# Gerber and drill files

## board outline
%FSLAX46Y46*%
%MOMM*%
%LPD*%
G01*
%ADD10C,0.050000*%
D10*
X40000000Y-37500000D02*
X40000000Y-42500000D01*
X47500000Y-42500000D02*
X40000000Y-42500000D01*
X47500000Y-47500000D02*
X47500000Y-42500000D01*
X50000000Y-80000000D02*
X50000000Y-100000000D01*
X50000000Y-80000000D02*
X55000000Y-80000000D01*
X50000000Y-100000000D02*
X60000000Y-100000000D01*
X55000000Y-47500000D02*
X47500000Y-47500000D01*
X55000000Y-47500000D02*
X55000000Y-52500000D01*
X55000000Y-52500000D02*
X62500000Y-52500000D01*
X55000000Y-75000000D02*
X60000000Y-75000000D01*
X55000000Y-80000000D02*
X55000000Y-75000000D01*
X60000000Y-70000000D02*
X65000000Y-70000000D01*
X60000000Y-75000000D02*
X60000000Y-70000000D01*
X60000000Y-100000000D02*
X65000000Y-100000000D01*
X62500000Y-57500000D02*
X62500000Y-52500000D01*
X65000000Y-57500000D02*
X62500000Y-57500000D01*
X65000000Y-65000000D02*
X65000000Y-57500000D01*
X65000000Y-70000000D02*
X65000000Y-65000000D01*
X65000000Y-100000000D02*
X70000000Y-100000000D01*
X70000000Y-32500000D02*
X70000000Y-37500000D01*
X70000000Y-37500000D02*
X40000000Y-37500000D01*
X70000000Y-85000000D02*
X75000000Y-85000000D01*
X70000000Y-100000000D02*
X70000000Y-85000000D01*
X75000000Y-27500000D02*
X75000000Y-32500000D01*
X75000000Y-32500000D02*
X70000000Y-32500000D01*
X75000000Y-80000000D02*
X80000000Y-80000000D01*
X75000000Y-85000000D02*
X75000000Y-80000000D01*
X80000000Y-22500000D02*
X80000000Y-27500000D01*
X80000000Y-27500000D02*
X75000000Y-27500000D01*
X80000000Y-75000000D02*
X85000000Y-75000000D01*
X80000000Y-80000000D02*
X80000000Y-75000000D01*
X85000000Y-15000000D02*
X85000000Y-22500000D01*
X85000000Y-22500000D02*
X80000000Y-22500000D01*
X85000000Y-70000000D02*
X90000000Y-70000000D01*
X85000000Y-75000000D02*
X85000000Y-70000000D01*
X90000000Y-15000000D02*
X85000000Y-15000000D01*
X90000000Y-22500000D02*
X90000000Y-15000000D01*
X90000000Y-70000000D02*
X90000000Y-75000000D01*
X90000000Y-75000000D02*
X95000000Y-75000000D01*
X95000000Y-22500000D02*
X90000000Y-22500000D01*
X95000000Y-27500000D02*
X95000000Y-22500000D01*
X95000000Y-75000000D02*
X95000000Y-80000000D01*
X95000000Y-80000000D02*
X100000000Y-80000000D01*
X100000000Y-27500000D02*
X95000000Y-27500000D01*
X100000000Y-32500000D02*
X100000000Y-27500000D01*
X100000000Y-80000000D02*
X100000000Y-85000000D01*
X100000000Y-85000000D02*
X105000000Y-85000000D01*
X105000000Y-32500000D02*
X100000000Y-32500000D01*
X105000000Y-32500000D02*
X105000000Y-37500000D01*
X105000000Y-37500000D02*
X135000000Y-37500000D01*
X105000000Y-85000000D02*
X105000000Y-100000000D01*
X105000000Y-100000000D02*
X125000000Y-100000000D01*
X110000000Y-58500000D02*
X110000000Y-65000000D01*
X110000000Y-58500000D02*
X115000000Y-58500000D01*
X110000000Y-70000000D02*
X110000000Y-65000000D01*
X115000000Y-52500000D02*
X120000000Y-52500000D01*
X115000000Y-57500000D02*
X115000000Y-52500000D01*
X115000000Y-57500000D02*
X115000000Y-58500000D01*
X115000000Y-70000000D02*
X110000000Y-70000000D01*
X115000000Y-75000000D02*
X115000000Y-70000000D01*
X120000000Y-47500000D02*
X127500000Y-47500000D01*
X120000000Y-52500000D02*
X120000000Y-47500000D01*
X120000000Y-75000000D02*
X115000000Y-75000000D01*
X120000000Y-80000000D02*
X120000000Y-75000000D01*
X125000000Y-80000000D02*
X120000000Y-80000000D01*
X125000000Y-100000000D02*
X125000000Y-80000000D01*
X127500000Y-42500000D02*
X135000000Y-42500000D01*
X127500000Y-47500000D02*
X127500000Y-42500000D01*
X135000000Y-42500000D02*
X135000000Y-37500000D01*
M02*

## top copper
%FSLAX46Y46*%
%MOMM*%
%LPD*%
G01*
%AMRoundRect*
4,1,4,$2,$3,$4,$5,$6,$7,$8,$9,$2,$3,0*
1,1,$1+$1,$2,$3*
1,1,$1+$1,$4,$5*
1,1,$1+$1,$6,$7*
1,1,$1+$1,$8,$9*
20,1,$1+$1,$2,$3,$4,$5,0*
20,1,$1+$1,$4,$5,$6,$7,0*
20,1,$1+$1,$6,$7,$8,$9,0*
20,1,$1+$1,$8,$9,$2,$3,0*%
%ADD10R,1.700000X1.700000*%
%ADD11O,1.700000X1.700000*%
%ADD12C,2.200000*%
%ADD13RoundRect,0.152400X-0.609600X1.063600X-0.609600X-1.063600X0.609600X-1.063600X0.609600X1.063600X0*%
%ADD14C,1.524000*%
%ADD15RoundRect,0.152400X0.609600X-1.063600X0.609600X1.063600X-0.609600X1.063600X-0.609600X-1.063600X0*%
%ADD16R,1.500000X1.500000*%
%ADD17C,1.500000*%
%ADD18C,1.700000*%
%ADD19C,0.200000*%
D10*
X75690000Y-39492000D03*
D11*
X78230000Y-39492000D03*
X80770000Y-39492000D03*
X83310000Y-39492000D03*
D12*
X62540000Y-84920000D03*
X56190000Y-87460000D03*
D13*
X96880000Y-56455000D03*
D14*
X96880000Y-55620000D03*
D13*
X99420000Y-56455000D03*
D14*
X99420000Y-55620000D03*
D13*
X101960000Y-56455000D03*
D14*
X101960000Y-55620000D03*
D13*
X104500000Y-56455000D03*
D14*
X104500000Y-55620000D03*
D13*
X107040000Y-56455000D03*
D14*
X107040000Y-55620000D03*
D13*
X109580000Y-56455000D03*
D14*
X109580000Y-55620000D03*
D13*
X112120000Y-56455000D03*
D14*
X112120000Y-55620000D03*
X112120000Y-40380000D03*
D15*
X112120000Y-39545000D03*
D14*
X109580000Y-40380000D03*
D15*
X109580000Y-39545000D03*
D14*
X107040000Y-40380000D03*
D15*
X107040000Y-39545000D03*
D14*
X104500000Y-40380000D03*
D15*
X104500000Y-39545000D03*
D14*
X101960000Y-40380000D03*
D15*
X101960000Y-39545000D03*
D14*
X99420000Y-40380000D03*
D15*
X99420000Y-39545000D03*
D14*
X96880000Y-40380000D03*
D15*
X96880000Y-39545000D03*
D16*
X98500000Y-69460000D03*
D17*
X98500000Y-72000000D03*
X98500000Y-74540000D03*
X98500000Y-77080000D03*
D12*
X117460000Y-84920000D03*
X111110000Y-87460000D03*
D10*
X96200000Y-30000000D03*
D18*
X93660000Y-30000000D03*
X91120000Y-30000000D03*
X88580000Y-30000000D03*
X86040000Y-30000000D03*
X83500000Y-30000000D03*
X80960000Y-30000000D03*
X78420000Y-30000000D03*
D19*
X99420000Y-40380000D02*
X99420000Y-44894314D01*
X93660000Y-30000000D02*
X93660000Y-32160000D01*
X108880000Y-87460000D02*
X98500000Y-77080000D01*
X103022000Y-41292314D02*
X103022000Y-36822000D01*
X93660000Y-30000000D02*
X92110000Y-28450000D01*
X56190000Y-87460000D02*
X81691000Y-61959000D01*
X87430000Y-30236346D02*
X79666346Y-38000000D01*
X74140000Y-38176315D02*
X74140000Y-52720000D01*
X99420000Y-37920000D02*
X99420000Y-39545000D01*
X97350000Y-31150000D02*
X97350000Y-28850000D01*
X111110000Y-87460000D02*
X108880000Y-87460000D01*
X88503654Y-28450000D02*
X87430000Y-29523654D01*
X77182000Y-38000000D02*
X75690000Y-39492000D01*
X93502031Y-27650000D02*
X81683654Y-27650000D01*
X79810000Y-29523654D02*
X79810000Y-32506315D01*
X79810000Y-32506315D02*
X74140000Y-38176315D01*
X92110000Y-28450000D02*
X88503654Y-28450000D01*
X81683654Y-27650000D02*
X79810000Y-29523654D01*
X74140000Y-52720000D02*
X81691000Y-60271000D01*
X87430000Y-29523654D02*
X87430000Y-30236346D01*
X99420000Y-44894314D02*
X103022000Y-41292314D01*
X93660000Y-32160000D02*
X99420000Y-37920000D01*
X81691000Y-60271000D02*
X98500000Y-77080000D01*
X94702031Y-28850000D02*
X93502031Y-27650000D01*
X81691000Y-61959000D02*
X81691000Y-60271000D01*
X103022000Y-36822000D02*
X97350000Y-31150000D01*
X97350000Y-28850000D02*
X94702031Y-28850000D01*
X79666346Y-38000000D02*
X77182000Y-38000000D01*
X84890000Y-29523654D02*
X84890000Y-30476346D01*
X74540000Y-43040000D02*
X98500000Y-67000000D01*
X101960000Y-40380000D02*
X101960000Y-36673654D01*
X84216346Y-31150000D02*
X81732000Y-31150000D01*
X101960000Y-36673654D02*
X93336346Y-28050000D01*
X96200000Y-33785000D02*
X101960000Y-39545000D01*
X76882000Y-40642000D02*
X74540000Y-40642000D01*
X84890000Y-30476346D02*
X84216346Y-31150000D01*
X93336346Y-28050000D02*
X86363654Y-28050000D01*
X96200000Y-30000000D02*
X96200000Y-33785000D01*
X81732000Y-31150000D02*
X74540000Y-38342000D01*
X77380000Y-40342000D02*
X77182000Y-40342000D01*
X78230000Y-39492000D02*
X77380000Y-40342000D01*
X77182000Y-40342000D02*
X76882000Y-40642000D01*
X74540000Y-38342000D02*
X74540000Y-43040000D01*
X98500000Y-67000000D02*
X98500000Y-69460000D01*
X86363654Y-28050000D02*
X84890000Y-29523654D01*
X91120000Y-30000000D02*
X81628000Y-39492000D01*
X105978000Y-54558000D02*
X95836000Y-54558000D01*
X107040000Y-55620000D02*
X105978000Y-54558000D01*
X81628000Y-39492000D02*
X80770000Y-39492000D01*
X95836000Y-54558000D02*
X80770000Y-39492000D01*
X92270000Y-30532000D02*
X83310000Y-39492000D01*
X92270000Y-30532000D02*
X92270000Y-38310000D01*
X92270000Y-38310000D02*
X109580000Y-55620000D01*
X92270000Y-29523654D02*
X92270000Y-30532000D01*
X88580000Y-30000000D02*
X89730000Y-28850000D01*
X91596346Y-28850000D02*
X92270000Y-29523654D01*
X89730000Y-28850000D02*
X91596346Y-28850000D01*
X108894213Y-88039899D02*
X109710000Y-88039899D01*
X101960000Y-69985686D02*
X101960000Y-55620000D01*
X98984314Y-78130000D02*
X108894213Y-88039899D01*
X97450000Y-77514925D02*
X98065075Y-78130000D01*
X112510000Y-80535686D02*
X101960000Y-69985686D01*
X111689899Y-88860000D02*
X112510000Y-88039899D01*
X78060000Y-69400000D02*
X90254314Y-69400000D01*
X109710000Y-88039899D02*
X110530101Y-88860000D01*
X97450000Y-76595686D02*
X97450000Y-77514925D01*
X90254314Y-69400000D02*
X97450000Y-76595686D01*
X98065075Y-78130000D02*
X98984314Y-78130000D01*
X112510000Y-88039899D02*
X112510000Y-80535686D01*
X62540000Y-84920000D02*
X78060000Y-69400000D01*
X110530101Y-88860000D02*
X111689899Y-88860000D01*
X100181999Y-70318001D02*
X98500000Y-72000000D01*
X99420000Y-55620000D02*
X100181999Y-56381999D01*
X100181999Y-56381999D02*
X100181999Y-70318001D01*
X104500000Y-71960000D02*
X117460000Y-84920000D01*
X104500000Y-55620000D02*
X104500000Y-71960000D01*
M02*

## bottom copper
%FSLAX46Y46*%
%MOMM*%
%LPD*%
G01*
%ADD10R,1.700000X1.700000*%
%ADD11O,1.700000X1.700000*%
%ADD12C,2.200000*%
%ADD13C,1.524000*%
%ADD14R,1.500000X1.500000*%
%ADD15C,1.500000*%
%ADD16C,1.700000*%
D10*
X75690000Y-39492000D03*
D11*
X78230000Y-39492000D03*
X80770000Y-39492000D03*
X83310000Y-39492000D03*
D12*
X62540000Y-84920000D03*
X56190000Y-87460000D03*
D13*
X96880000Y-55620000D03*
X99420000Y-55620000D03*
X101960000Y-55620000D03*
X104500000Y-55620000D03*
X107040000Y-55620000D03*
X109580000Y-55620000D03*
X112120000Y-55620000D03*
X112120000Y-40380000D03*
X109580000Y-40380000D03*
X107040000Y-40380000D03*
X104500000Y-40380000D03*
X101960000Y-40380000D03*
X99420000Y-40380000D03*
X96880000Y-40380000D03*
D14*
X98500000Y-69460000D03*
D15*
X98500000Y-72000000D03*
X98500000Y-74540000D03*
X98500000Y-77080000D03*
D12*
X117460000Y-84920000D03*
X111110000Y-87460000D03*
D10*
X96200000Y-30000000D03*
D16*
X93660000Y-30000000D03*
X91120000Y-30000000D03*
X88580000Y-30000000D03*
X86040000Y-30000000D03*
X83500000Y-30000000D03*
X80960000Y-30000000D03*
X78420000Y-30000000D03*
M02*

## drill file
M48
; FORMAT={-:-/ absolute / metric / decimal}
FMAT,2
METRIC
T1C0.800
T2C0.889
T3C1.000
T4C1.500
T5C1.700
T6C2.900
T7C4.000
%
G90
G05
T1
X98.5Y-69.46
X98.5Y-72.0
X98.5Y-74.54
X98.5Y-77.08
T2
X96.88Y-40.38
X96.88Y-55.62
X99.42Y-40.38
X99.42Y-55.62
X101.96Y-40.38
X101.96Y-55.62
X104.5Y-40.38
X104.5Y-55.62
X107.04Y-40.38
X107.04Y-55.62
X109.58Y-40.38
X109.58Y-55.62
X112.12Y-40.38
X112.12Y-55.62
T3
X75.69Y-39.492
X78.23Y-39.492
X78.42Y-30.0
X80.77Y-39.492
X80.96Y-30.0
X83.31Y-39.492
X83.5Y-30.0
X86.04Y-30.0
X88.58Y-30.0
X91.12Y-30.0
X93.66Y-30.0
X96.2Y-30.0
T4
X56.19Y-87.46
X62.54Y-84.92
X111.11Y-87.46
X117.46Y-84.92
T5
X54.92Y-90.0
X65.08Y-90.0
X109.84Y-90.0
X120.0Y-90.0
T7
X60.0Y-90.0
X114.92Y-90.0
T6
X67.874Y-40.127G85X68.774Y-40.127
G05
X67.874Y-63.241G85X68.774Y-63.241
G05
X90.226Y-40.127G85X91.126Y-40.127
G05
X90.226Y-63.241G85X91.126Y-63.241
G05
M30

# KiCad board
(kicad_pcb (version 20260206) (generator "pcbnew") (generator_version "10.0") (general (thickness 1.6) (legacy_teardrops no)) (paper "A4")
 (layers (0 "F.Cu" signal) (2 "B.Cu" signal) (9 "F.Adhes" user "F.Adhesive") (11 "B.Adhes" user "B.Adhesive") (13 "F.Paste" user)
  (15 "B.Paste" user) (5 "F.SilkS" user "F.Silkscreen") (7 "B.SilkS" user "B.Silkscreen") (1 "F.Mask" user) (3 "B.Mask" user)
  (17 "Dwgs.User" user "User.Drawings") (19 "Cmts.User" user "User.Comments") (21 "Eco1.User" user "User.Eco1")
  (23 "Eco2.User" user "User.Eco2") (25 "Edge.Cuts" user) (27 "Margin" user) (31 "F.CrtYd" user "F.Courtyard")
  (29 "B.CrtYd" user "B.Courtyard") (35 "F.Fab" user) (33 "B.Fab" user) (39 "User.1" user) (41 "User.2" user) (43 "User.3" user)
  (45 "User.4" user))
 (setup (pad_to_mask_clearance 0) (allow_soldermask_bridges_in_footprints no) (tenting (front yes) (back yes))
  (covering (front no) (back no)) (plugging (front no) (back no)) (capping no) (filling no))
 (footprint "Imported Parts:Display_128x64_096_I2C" (layer "F.Cu") (at 79.5 39.492)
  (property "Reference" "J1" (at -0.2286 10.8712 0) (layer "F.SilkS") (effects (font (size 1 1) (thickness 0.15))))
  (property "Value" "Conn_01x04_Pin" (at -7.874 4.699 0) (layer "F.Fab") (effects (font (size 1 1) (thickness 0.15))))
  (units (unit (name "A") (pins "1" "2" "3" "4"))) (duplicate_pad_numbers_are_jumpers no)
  (pad "" np_thru_hole oval (at -11.176 0.635) (size 3.8 2.9) (drill oval 3.8 2.9) (layers "*.Cu" "*.Mask"))
  (pad "" np_thru_hole oval (at -11.176 23.749) (size 3.8 2.9) (drill oval 3.8 2.9) (layers "*.Cu" "*.Mask"))
  (pad "" np_thru_hole oval (at 11.176 0.635) (size 3.8 2.9) (drill oval 3.8 2.9) (layers "*.Cu" "*.Mask"))
  (pad "" np_thru_hole oval (at 11.176 23.749) (size 3.8 2.9) (drill oval 3.8 2.9) (layers "*.Cu" "*.Mask"))
  (pad "1" thru_hole rect (at -3.81 0 90) (size 1.7 1.7) (drill 1) (layers "*.Cu" "*.Mask") (remove_unused_layers no) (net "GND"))
  (pad "2" thru_hole oval (at -1.27 0 90) (size 1.7 1.7) (drill 1) (layers "*.Cu" "*.Mask") (remove_unused_layers no) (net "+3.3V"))
  (pad "3" thru_hole oval (at 1.27 0 90) (size 1.7 1.7) (drill 1) (layers "*.Cu" "*.Mask") (remove_unused_layers no) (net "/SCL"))
  (pad "4" thru_hole oval (at 3.81 0 90) (size 1.7 1.7) (drill 1) (layers "*.Cu" "*.Mask") (remove_unused_layers no) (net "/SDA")))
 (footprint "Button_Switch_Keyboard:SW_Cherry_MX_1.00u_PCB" (layer "F.Cu") (at 62.54 84.92)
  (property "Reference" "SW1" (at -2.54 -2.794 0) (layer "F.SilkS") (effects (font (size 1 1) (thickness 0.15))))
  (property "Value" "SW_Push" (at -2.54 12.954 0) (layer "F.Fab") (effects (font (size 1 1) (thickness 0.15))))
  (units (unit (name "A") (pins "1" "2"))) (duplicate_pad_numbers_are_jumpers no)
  (pad "" np_thru_hole circle (at -7.62 5.08) (size 1.7 1.7) (drill 1.7) (layers "*.Cu" "*.Mask"))
  (pad "" np_thru_hole circle (at -2.54 5.08) (size 4 4) (drill 4) (layers "*.Cu" "*.Mask"))
  (pad "" np_thru_hole circle (at 2.54 5.08) (size 1.7 1.7) (drill 1.7) (layers "*.Cu" "*.Mask"))
  (pad "1" thru_hole circle (at 0 0) (size 2.2 2.2) (drill 1.5) (layers "*.Cu" "*.Mask") (remove_unused_layers no) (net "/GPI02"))
  (pad "2" thru_hole circle (at -6.35 2.54) (size 2.2 2.2) (drill 1.5) (layers "*.Cu" "*.Mask") (remove_unused_layers no) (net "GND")))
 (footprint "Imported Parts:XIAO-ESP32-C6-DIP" (layer "F.Cu") (at 104.5 48 180)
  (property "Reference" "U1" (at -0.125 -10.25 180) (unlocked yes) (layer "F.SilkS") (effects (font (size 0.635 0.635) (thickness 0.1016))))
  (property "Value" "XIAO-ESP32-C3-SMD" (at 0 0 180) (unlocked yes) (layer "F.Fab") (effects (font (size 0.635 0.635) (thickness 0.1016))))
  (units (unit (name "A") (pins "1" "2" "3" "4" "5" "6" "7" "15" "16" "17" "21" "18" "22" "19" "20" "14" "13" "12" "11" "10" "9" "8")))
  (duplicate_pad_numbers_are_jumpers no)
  (pad "1" smd roundrect (at 7.62 -8.455 270) (size 2.432 1.524) (layers "F.Cu" "F.Mask") (roundrect_rratio 0.1)
   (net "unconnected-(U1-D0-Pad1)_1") (thermal_bridge_angle 45))
  (pad "1" thru_hole circle (at 7.62 -7.62 270) (size 1.524 1.524) (drill 0.889) (layers "*.Cu" "*.Mask") (remove_unused_layers no)
   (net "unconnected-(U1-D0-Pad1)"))
  (pad "2" smd roundrect (at 5.08 -8.455 270) (size 2.432 1.524) (layers "F.Cu" "F.Mask") (roundrect_rratio 0.1) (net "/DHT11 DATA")
   (thermal_bridge_angle 45))
  (pad "2" thru_hole circle (at 5.08 -7.62 270) (size 1.524 1.524) (drill 0.889) (layers "*.Cu" "*.Mask") (remove_unused_layers no)
   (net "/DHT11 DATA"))
  (pad "3" smd roundrect (at 2.54 -8.455 270) (size 2.432 1.524) (layers "F.Cu" "F.Mask") (roundrect_rratio 0.1) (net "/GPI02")
   (thermal_bridge_angle 45))
  (pad "3" thru_hole circle (at 2.54 -7.62 270) (size 1.524 1.524) (drill 0.889) (layers "*.Cu" "*.Mask") (remove_unused_layers no)
   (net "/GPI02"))
  (pad "4" smd roundrect (at 0 -8.455 270) (size 2.432 1.524) (layers "F.Cu" "F.Mask") (roundrect_rratio 0.1) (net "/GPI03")
   (thermal_bridge_angle 45))
  (pad "4" thru_hole circle (at 0 -7.62 270) (size 1.524 1.524) (drill 0.889) (layers "*.Cu" "*.Mask") (remove_unused_layers no)
   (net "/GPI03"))
  (pad "5" smd roundrect (at -2.54 -8.455 270) (size 2.432 1.524) (layers "F.Cu" "F.Mask") (roundrect_rratio 0.1) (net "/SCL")
   (thermal_bridge_angle 45))
  (pad "5" thru_hole circle (at -2.54 -7.62 270) (size 1.524 1.524) (drill 0.889) (layers "*.Cu" "*.Mask") (remove_unused_layers no)
   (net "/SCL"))
  (pad "6" smd roundrect (at -5.08 -8.455 270) (size 2.432 1.524) (layers "F.Cu" "F.Mask") (roundrect_rratio 0.1) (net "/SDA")
   (thermal_bridge_angle 45))
  (pad "6" thru_hole circle (at -5.08 -7.62 270) (size 1.524 1.524) (drill 0.889) (layers "*.Cu" "*.Mask") (remove_unused_layers no)
   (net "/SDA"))
  (pad "7" smd roundrect (at -7.62 -8.455 270) (size 2.432 1.524) (layers "F.Cu" "F.Mask") (roundrect_rratio 0.1)
   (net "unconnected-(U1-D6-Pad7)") (thermal_bridge_angle 45))
  (pad "7" thru_hole circle (at -7.62 -7.62 270) (size 1.524 1.524) (drill 0.889) (layers "*.Cu" "*.Mask") (remove_unused_layers no)
   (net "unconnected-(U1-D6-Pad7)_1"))
  (pad "8" thru_hole circle (at -7.62 7.62 90) (size 1.524 1.524) (drill 0.889) (layers "*.Cu" "*.Mask") (remove_unused_layers no)
   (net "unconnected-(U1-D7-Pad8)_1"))
  (pad "8" smd roundrect (at -7.62 8.455 90) (size 2.432 1.524) (layers "F.Cu" "F.Mask") (roundrect_rratio 0.1)
   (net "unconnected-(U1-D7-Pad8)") (thermal_bridge_angle 45))
  (pad "9" thru_hole circle (at -5.08 7.62 90) (size 1.524 1.524) (drill 0.889) (layers "*.Cu" "*.Mask") (remove_unused_layers no)
   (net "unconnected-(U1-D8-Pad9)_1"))
  (pad "9" smd roundrect (at -5.08 8.455 90) (size 2.432 1.524) (layers "F.Cu" "F.Mask") (roundrect_rratio 0.1)
   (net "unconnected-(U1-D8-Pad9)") (thermal_bridge_angle 45))
  (pad "10" thru_hole circle (at -2.54 7.62 90) (size 1.524 1.524) (drill 0.889) (layers "*.Cu" "*.Mask") (remove_unused_layers no)
   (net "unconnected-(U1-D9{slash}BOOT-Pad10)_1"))
  (pad "10" smd roundrect (at -2.54 8.455 90) (size 2.432 1.524) (layers "F.Cu" "F.Mask") (roundrect_rratio 0.1)
   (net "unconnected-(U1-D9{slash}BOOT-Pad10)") (thermal_bridge_angle 45))
  (pad "11" thru_hole circle (at 0 7.62 90) (size 1.524 1.524) (drill 0.889) (layers "*.Cu" "*.Mask") (remove_unused_layers no)
   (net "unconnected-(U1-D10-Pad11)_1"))
  (pad "11" smd roundrect (at 0 8.455 90) (size 2.432 1.524) (layers "F.Cu" "F.Mask") (roundrect_rratio 0.1)
   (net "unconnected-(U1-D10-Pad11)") (thermal_bridge_angle 45))
  (pad "12" thru_hole circle (at 2.54 7.62 90) (size 1.524 1.524) (drill 0.889) (layers "*.Cu" "*.Mask") (remove_unused_layers no)
   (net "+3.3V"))
  (pad "12" smd roundrect (at 2.54 8.455 90) (size 2.432 1.524) (layers "F.Cu" "F.Mask") (roundrect_rratio 0.1) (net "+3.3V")
   (thermal_bridge_angle 45))
  (pad "13" thru_hole circle (at 5.08 7.62 90) (size 1.524 1.524) (drill 0.889) (layers "*.Cu" "*.Mask") (remove_unused_layers no)
   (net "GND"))
  (pad "13" smd roundrect (at 5.08 8.455 90) (size 2.432 1.524) (layers "F.Cu" "F.Mask") (roundrect_rratio 0.1) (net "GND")
   (thermal_bridge_angle 45))
  (pad "14" thru_hole circle (at 7.62 7.62 90) (size 1.524 1.524) (drill 0.889) (layers "*.Cu" "*.Mask") (remove_unused_layers no)
   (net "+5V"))
  (pad "14" smd roundrect (at 7.62 8.455 90) (size 2.432 1.524) (layers "F.Cu" "F.Mask") (roundrect_rratio 0.1) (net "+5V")
   (thermal_bridge_angle 45)))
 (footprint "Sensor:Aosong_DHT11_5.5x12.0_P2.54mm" (layer "F.Cu") (at 98.5 69.46)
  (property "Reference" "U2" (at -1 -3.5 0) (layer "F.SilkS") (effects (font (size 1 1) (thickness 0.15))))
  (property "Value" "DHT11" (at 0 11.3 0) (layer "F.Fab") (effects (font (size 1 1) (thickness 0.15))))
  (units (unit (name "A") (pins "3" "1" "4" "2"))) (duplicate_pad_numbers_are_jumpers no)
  (pad "1" thru_hole rect (at 0 0) (size 1.5 1.5) (drill 0.8) (layers "*.Cu" "*.Mask") (remove_unused_layers no) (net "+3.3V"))
  (pad "2" thru_hole circle (at 0 2.54) (size 1.5 1.5) (drill 0.8) (layers "*.Cu" "*.Mask") (remove_unused_layers no) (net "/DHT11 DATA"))
  (pad "3" thru_hole circle (at 0 5.08) (size 1.5 1.5) (drill 0.8) (layers "*.Cu" "*.Mask") (remove_unused_layers no)
   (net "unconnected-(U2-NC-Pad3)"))
  (pad "4" thru_hole circle (at 0 7.62) (size 1.5 1.5) (drill 0.8) (layers "*.Cu" "*.Mask") (remove_unused_layers no) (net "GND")))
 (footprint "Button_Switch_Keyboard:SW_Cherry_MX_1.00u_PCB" (layer "F.Cu") (at 117.46 84.92)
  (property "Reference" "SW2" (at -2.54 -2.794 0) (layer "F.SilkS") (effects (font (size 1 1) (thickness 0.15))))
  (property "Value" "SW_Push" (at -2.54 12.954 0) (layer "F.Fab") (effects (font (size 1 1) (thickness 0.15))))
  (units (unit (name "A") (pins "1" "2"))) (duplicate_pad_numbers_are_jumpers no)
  (pad "" np_thru_hole circle (at -7.62 5.08) (size 1.7 1.7) (drill 1.7) (layers "*.Cu" "*.Mask"))
  (pad "" np_thru_hole circle (at -2.54 5.08) (size 4 4) (drill 4) (layers "*.Cu" "*.Mask"))
  (pad "" np_thru_hole circle (at 2.54 5.08) (size 1.7 1.7) (drill 1.7) (layers "*.Cu" "*.Mask"))
  (pad "1" thru_hole circle (at 0 0) (size 2.2 2.2) (drill 1.5) (layers "*.Cu" "*.Mask") (remove_unused_layers no) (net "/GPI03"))
  (pad "2" thru_hole circle (at -6.35 2.54) (size 2.2 2.2) (drill 1.5) (layers "*.Cu" "*.Mask") (remove_unused_layers no) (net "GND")))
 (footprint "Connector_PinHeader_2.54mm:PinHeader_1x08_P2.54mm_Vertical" (layer "F.Cu") (at 96.2 30 -90)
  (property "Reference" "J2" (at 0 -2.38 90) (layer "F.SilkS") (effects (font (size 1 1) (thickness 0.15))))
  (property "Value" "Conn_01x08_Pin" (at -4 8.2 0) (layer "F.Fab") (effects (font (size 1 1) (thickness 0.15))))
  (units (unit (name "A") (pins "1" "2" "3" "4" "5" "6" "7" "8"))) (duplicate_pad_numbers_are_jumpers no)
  (pad "1" thru_hole rect (at 0 0 270) (size 1.7 1.7) (drill 1) (layers "*.Cu" "*.Mask") (remove_unused_layers no) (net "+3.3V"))
  (pad "2" thru_hole circle (at 0 2.54 270) (size 1.7 1.7) (drill 1) (layers "*.Cu" "*.Mask") (remove_unused_layers no) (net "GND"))
  (pad "3" thru_hole circle (at 0 5.08 270) (size 1.7 1.7) (drill 1) (layers "*.Cu" "*.Mask") (remove_unused_layers no) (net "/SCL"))
  (pad "4" thru_hole circle (at 0 7.62 270) (size 1.7 1.7) (drill 1) (layers "*.Cu" "*.Mask") (remove_unused_layers no) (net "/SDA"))
  (pad "5" thru_hole circle (at 0 10.16 270) (size 1.7 1.7) (drill 1) (layers "*.Cu" "*.Mask") (remove_unused_layers no)
   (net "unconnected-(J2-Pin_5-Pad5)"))
  (pad "6" thru_hole circle (at 0 12.7 270) (size 1.7 1.7) (drill 1) (layers "*.Cu" "*.Mask") (remove_unused_layers no)
   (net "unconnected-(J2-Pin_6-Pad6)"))
  (pad "7" thru_hole circle (at 0 15.24 270) (size 1.7 1.7) (drill 1) (layers "*.Cu" "*.Mask") (remove_unused_layers no)
   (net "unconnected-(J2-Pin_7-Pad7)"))
  (pad "8" thru_hole circle (at 0 17.78 270) (size 1.7 1.7) (drill 1) (layers "*.Cu" "*.Mask") (remove_unused_layers no)
   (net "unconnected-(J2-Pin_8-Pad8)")))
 (gr_line (start 40 37.5) (end 40 42.5) (stroke (width 0.05) (type default)) (layer "Edge.Cuts"))
 (gr_line (start 47.5 42.5) (end 40 42.5) (stroke (width 0.05) (type default)) (layer "Edge.Cuts"))
 (gr_line (start 47.5 47.5) (end 47.5 42.5) (stroke (width 0.05) (type default)) (layer "Edge.Cuts"))
 (gr_line (start 50 80) (end 50 100) (stroke (width 0.05) (type default)) (layer "Edge.Cuts"))
 (gr_line (start 50 80) (end 55 80) (stroke (width 0.05) (type default)) (layer "Edge.Cuts"))
 (gr_line (start 50 100) (end 60 100) (stroke (width 0.05) (type default)) (layer "Edge.Cuts"))
 (gr_line (start 55 47.5) (end 47.5 47.5) (stroke (width 0.05) (type default)) (layer "Edge.Cuts"))
 (gr_line (start 55 47.5) (end 55 52.5) (stroke (width 0.05) (type default)) (layer "Edge.Cuts"))
 (gr_line (start 55 52.5) (end 62.5 52.5) (stroke (width 0.05) (type default)) (layer "Edge.Cuts"))
 (gr_line (start 55 75) (end 60 75) (stroke (width 0.05) (type default)) (layer "Edge.Cuts"))
 (gr_line (start 55 80) (end 55 75) (stroke (width 0.05) (type default)) (layer "Edge.Cuts"))
 (gr_line (start 60 70) (end 65 70) (stroke (width 0.05) (type default)) (layer "Edge.Cuts"))
 (gr_line (start 60 75) (end 60 70) (stroke (width 0.05) (type default)) (layer "Edge.Cuts"))
 (gr_line (start 60 100) (end 65 100) (stroke (width 0.05) (type default)) (layer "Edge.Cuts"))
 (gr_line (start 62.5 57.5) (end 62.5 52.5) (stroke (width 0.05) (type default)) (layer "Edge.Cuts"))
 (gr_line (start 65 57.5) (end 62.5 57.5) (stroke (width 0.05) (type default)) (layer "Edge.Cuts"))
 (gr_line (start 65 65) (end 65 57.5) (stroke (width 0.05) (type default)) (layer "Edge.Cuts"))
 (gr_line (start 65 70) (end 65 65) (stroke (width 0.05) (type default)) (layer "Edge.Cuts"))
 (gr_line (start 65 100) (end 70 100) (stroke (width 0.05) (type default)) (layer "Edge.Cuts"))
 (gr_line (start 70 32.5) (end 70 37.5) (stroke (width 0.05) (type default)) (layer "Edge.Cuts"))
 (gr_line (start 70 37.5) (end 40 37.5) (stroke (width 0.05) (type default)) (layer "Edge.Cuts"))
 (gr_line (start 70 85) (end 75 85) (stroke (width 0.05) (type default)) (layer "Edge.Cuts"))
 (gr_line (start 70 100) (end 70 85) (stroke (width 0.05) (type default)) (layer "Edge.Cuts"))
 (gr_line (start 75 27.5) (end 75 32.5) (stroke (width 0.05) (type default)) (layer "Edge.Cuts"))
 (gr_line (start 75 32.5) (end 70 32.5) (stroke (width 0.05) (type default)) (layer "Edge.Cuts"))
 (gr_line (start 75 80) (end 80 80) (stroke (width 0.05) (type default)) (layer "Edge.Cuts"))
 (gr_line (start 75 85) (end 75 80) (stroke (width 0.05) (type default)) (layer "Edge.Cuts"))
 (gr_line (start 80 22.5) (end 80 27.5) (stroke (width 0.05) (type default)) (layer "Edge.Cuts"))
 (gr_line (start 80 27.5) (end 75 27.5) (stroke (width 0.05) (type default)) (layer "Edge.Cuts"))
 (gr_line (start 80 75) (end 85 75) (stroke (width 0.05) (type default)) (layer "Edge.Cuts"))
 (gr_line (start 80 80) (end 80 75) (stroke (width 0.05) (type default)) (layer "Edge.Cuts"))
 (gr_line (start 85 15) (end 85 22.5) (stroke (width 0.05) (type default)) (layer "Edge.Cuts"))
 (gr_line (start 85 22.5) (end 80 22.5) (stroke (width 0.05) (type default)) (layer "Edge.Cuts"))
 (gr_line (start 85 70) (end 90 70) (stroke (width 0.05) (type default)) (layer "Edge.Cuts"))
 (gr_line (start 85 75) (end 85 70) (stroke (width 0.05) (type default)) (layer "Edge.Cuts"))
 (gr_line (start 90 15) (end 85 15) (stroke (width 0.05) (type default)) (layer "Edge.Cuts"))
 (gr_line (start 90 22.5) (end 90 15) (stroke (width 0.05) (type default)) (layer "Edge.Cuts"))
 (gr_line (start 90 70) (end 90 75) (stroke (width 0.05) (type default)) (layer "Edge.Cuts"))
 (gr_line (start 90 75) (end 95 75) (stroke (width 0.05) (type default)) (layer "Edge.Cuts"))
 (gr_line (start 95 22.5) (end 90 22.5) (stroke (width 0.05) (type default)) (layer "Edge.Cuts"))
 (gr_line (start 95 27.5) (end 95 22.5) (stroke (width 0.05) (type default)) (layer "Edge.Cuts"))
 (gr_line (start 95 75) (end 95 80) (stroke (width 0.05) (type default)) (layer "Edge.Cuts"))
 (gr_line (start 95 80) (end 100 80) (stroke (width 0.05) (type default)) (layer "Edge.Cuts"))
 (gr_line (start 100 27.5) (end 95 27.5) (stroke (width 0.05) (type default)) (layer "Edge.Cuts"))
 (gr_line (start 100 32.5) (end 100 27.5) (stroke (width 0.05) (type default)) (layer "Edge.Cuts"))
 (gr_line (start 100 80) (end 100 85) (stroke (width 0.05) (type default)) (layer "Edge.Cuts"))
 (gr_line (start 100 85) (end 105 85) (stroke (width 0.05) (type default)) (layer "Edge.Cuts"))
 (gr_line (start 105 32.5) (end 100 32.5) (stroke (width 0.05) (type default)) (layer "Edge.Cuts"))
 (gr_line (start 105 32.5) (end 105 37.5) (stroke (width 0.05) (type default)) (layer "Edge.Cuts"))
 (gr_line (start 105 37.5) (end 135 37.5) (stroke (width 0.05) (type default)) (layer "Edge.Cuts"))
 (gr_line (start 105 85) (end 105 100) (stroke (width 0.05) (type default)) (layer "Edge.Cuts"))
 (gr_line (start 105 100) (end 125 100) (stroke (width 0.05) (type default)) (layer "Edge.Cuts"))
 (gr_line (start 110 58.5) (end 110 65) (stroke (width 0.05) (type default)) (layer "Edge.Cuts"))
 (gr_line (start 110 58.5) (end 115 58.5) (stroke (width 0.05) (type default)) (layer "Edge.Cuts"))
 (gr_line (start 110 70) (end 110 65) (stroke (width 0.05) (type default)) (layer "Edge.Cuts"))
 (gr_line (start 115 52.5) (end 120 52.5) (stroke (width 0.05) (type default)) (layer "Edge.Cuts"))
 (gr_line (start 115 57.5) (end 115 52.5) (stroke (width 0.05) (type default)) (layer "Edge.Cuts"))
 (gr_line (start 115 57.5) (end 115 58.5) (stroke (width 0.05) (type default)) (layer "Edge.Cuts"))
 (gr_line (start 115 70) (end 110 70) (stroke (width 0.05) (type default)) (layer "Edge.Cuts"))
 (gr_line (start 115 75) (end 115 70) (stroke (width 0.05) (type default)) (layer "Edge.Cuts"))
 (gr_line (start 120 47.5) (end 127.5 47.5) (stroke (width 0.05) (type default)) (layer "Edge.Cuts"))
 (gr_line (start 120 52.5) (end 120 47.5) (stroke (width 0.05) (type default)) (layer "Edge.Cuts"))
 (gr_line (start 120 75) (end 115 75) (stroke (width 0.05) (type default)) (layer "Edge.Cuts"))
 (gr_line (start 120 80) (end 120 75) (stroke (width 0.05) (type default)) (layer "Edge.Cuts"))
 (gr_line (start 125 80) (end 120 80) (stroke (width 0.05) (type default)) (layer "Edge.Cuts"))
 (gr_line (start 125 100) (end 125 80) (stroke (width 0.05) (type default)) (layer "Edge.Cuts"))
 (gr_line (start 127.5 42.5) (end 135 42.5) (stroke (width 0.05) (type default)) (layer "Edge.Cuts"))
 (gr_line (start 127.5 47.5) (end 127.5 42.5) (stroke (width 0.05) (type default)) (layer "Edge.Cuts"))
 (gr_line (start 135 42.5) (end 135 37.5) (stroke (width 0.05) (type default)) (layer "Edge.Cuts"))
 (segment (start 99.42 40.38) (end 99.42 44.894314) (width 0.2) (layer "F.Cu") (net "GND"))
 (segment (start 93.66 30) (end 93.66 32.16) (width 0.2) (layer "F.Cu") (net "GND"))
 (segment (start 108.88 87.46) (end 98.5 77.08) (width 0.2) (layer "F.Cu") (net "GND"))
 (segment (start 103.022 41.292314) (end 103.022 36.822) (width 0.2) (layer "F.Cu") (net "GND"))
 (segment (start 93.66 30) (end 92.11 28.45) (width 0.2) (layer "F.Cu") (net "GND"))
 (segment (start 56.19 87.46) (end 81.691 61.959) (width 0.2) (layer "F.Cu") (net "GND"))
 (segment (start 87.43 30.236346) (end 79.666346 38) (width 0.2) (layer "F.Cu") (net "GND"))
 (segment (start 74.14 38.176315) (end 74.14 52.72) (width 0.2) (layer "F.Cu") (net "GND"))
 (segment (start 99.42 37.92) (end 99.42 39.545) (width 0.2) (layer "F.Cu") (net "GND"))
 (segment (start 97.35 31.15) (end 97.35 28.85) (width 0.2) (layer "F.Cu") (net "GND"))
 (segment (start 111.11 87.46) (end 108.88 87.46) (width 0.2) (layer "F.Cu") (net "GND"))
 (segment (start 88.503654 28.45) (end 87.43 29.523654) (width 0.2) (layer "F.Cu") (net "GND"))
 (segment (start 77.182 38) (end 75.69 39.492) (width 0.2) (layer "F.Cu") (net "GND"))
 (segment (start 93.502031 27.65) (end 81.683654 27.65) (width 0.2) (layer "F.Cu") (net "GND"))
 (segment (start 79.81 29.523654) (end 79.81 32.506315) (width 0.2) (layer "F.Cu") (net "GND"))
 (segment (start 79.81 32.506315) (end 74.14 38.176315) (width 0.2) (layer "F.Cu") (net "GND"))
 (segment (start 92.11 28.45) (end 88.503654 28.45) (width 0.2) (layer "F.Cu") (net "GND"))
 (segment (start 81.683654 27.65) (end 79.81 29.523654) (width 0.2) (layer "F.Cu") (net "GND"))
 (segment (start 74.14 52.72) (end 81.691 60.271) (width 0.2) (layer "F.Cu") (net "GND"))
 (segment (start 87.43 29.523654) (end 87.43 30.236346) (width 0.2) (layer "F.Cu") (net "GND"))
 (segment (start 99.42 44.894314) (end 103.022 41.292314) (width 0.2) (layer "F.Cu") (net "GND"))
 (segment (start 93.66 32.16) (end 99.42 37.92) (width 0.2) (layer "F.Cu") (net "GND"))
 (segment (start 81.691 60.271) (end 98.5 77.08) (width 0.2) (layer "F.Cu") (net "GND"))
 (segment (start 94.702031 28.85) (end 93.502031 27.65) (width 0.2) (layer "F.Cu") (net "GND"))
 (segment (start 81.691 61.959) (end 81.691 60.271) (width 0.2) (layer "F.Cu") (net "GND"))
 (segment (start 103.022 36.822) (end 97.35 31.15) (width 0.2) (layer "F.Cu") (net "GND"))
 (segment (start 97.35 28.85) (end 94.702031 28.85) (width 0.2) (layer "F.Cu") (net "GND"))
 (segment (start 79.666346 38) (end 77.182 38) (width 0.2) (layer "F.Cu") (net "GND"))
 (segment (start 84.89 29.523654) (end 84.89 30.476346) (width 0.2) (layer "F.Cu") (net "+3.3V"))
 (segment (start 74.54 43.04) (end 98.5 67) (width 0.2) (layer "F.Cu") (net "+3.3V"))
 (segment (start 101.96 40.38) (end 101.96 36.673654) (width 0.2) (layer "F.Cu") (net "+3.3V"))
 (segment (start 84.216346 31.15) (end 81.732 31.15) (width 0.2) (layer "F.Cu") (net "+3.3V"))
 (segment (start 101.96 36.673654) (end 93.336346 28.05) (width 0.2) (layer "F.Cu") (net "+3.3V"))
 (segment (start 96.2 33.785) (end 101.96 39.545) (width 0.2) (layer "F.Cu") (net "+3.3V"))
 (segment (start 76.882 40.642) (end 74.54 40.642) (width 0.2) (layer "F.Cu") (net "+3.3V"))
 (segment (start 84.89 30.476346) (end 84.216346 31.15) (width 0.2) (layer "F.Cu") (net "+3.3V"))
 (segment (start 93.336346 28.05) (end 86.363654 28.05) (width 0.2) (layer "F.Cu") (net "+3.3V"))
 (segment (start 96.2 30) (end 96.2 33.785) (width 0.2) (layer "F.Cu") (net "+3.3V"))
 (segment (start 81.732 31.15) (end 74.54 38.342) (width 0.2) (layer "F.Cu") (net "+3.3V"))
 (segment (start 77.38 40.342) (end 77.182 40.342) (width 0.2) (layer "F.Cu") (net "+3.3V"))
 (segment (start 78.23 39.492) (end 77.38 40.342) (width 0.2) (layer "F.Cu") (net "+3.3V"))
 (segment (start 77.182 40.342) (end 76.882 40.642) (width 0.2) (layer "F.Cu") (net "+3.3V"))
 (segment (start 74.54 38.342) (end 74.54 43.04) (width 0.2) (layer "F.Cu") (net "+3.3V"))
 (segment (start 98.5 67) (end 98.5 69.46) (width 0.2) (layer "F.Cu") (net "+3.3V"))
 (segment (start 86.363654 28.05) (end 84.89 29.523654) (width 0.2) (layer "F.Cu") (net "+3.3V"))
 (segment (start 91.12 30) (end 81.628 39.492) (width 0.2) (layer "F.Cu") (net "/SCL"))
 (segment (start 105.978 54.558) (end 95.836 54.558) (width 0.2) (layer "F.Cu") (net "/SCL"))
 (segment (start 107.04 55.62) (end 105.978 54.558) (width 0.2) (layer "F.Cu") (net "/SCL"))
 (segment (start 81.628 39.492) (end 80.77 39.492) (width 0.2) (layer "F.Cu") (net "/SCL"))
 (segment (start 95.836 54.558) (end 80.77 39.492) (width 0.2) (layer "F.Cu") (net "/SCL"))
 (segment (start 92.27 30.532) (end 83.31 39.492) (width 0.2) (layer "F.Cu") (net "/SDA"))
 (segment (start 92.27 30.532) (end 92.27 38.31) (width 0.2) (layer "F.Cu") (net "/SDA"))
 (segment (start 92.27 38.31) (end 109.58 55.62) (width 0.2) (layer "F.Cu") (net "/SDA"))
 (segment (start 92.27 29.523654) (end 92.27 30.532) (width 0.2) (layer "F.Cu") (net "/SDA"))
 (segment (start 88.58 30) (end 89.73 28.85) (width 0.2) (layer "F.Cu") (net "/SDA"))
 (segment (start 91.596346 28.85) (end 92.27 29.523654) (width 0.2) (layer "F.Cu") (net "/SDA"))
 (segment (start 89.73 28.85) (end 91.596346 28.85) (width 0.2) (layer "F.Cu") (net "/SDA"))
 (segment (start 108.894213 88.039899) (end 109.71 88.039899) (width 0.2) (layer "F.Cu") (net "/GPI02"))
 (segment (start 101.96 69.985686) (end 101.96 55.62) (width 0.2) (layer "F.Cu") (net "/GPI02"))
 (segment (start 98.984314 78.13) (end 108.894213 88.039899) (width 0.2) (layer "F.Cu") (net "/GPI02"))
 (segment (start 97.45 77.514925) (end 98.065075 78.13) (width 0.2) (layer "F.Cu") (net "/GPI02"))
 (segment (start 112.51 80.535686) (end 101.96 69.985686) (width 0.2) (layer "F.Cu") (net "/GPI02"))
 (segment (start 111.689899 88.86) (end 112.51 88.039899) (width 0.2) (layer "F.Cu") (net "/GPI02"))
 (segment (start 78.06 69.4) (end 90.254314 69.4) (width 0.2) (layer "F.Cu") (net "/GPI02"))
 (segment (start 109.71 88.039899) (end 110.530101 88.86) (width 0.2) (layer "F.Cu") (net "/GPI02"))
 (segment (start 97.45 76.595686) (end 97.45 77.514925) (width 0.2) (layer "F.Cu") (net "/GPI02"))
 (segment (start 90.254314 69.4) (end 97.45 76.595686) (width 0.2) (layer "F.Cu") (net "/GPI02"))
 (segment (start 98.065075 78.13) (end 98.984314 78.13) (width 0.2) (layer "F.Cu") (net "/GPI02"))
 (segment (start 112.51 88.039899) (end 112.51 80.535686) (width 0.2) (layer "F.Cu") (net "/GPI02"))
 (segment (start 62.54 84.92) (end 78.06 69.4) (width 0.2) (layer "F.Cu") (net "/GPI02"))
 (segment (start 110.530101 88.86) (end 111.689899 88.86) (width 0.2) (layer "F.Cu") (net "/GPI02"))
 (segment (start 100.181999 70.318001) (end 98.5 72) (width 0.2) (layer "F.Cu") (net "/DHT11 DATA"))
 (segment (start 99.42 55.62) (end 100.181999 56.381999) (width 0.2) (layer "F.Cu") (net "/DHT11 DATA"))
 (segment (start 100.181999 56.381999) (end 100.181999 70.318001) (width 0.2) (layer "F.Cu") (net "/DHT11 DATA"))
 (segment (start 104.5 71.96) (end 117.46 84.92) (width 0.2) (layer "F.Cu") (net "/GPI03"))
 (segment (start 104.5 55.62) (end 104.5 71.96) (width 0.2) (layer "F.Cu") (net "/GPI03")))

